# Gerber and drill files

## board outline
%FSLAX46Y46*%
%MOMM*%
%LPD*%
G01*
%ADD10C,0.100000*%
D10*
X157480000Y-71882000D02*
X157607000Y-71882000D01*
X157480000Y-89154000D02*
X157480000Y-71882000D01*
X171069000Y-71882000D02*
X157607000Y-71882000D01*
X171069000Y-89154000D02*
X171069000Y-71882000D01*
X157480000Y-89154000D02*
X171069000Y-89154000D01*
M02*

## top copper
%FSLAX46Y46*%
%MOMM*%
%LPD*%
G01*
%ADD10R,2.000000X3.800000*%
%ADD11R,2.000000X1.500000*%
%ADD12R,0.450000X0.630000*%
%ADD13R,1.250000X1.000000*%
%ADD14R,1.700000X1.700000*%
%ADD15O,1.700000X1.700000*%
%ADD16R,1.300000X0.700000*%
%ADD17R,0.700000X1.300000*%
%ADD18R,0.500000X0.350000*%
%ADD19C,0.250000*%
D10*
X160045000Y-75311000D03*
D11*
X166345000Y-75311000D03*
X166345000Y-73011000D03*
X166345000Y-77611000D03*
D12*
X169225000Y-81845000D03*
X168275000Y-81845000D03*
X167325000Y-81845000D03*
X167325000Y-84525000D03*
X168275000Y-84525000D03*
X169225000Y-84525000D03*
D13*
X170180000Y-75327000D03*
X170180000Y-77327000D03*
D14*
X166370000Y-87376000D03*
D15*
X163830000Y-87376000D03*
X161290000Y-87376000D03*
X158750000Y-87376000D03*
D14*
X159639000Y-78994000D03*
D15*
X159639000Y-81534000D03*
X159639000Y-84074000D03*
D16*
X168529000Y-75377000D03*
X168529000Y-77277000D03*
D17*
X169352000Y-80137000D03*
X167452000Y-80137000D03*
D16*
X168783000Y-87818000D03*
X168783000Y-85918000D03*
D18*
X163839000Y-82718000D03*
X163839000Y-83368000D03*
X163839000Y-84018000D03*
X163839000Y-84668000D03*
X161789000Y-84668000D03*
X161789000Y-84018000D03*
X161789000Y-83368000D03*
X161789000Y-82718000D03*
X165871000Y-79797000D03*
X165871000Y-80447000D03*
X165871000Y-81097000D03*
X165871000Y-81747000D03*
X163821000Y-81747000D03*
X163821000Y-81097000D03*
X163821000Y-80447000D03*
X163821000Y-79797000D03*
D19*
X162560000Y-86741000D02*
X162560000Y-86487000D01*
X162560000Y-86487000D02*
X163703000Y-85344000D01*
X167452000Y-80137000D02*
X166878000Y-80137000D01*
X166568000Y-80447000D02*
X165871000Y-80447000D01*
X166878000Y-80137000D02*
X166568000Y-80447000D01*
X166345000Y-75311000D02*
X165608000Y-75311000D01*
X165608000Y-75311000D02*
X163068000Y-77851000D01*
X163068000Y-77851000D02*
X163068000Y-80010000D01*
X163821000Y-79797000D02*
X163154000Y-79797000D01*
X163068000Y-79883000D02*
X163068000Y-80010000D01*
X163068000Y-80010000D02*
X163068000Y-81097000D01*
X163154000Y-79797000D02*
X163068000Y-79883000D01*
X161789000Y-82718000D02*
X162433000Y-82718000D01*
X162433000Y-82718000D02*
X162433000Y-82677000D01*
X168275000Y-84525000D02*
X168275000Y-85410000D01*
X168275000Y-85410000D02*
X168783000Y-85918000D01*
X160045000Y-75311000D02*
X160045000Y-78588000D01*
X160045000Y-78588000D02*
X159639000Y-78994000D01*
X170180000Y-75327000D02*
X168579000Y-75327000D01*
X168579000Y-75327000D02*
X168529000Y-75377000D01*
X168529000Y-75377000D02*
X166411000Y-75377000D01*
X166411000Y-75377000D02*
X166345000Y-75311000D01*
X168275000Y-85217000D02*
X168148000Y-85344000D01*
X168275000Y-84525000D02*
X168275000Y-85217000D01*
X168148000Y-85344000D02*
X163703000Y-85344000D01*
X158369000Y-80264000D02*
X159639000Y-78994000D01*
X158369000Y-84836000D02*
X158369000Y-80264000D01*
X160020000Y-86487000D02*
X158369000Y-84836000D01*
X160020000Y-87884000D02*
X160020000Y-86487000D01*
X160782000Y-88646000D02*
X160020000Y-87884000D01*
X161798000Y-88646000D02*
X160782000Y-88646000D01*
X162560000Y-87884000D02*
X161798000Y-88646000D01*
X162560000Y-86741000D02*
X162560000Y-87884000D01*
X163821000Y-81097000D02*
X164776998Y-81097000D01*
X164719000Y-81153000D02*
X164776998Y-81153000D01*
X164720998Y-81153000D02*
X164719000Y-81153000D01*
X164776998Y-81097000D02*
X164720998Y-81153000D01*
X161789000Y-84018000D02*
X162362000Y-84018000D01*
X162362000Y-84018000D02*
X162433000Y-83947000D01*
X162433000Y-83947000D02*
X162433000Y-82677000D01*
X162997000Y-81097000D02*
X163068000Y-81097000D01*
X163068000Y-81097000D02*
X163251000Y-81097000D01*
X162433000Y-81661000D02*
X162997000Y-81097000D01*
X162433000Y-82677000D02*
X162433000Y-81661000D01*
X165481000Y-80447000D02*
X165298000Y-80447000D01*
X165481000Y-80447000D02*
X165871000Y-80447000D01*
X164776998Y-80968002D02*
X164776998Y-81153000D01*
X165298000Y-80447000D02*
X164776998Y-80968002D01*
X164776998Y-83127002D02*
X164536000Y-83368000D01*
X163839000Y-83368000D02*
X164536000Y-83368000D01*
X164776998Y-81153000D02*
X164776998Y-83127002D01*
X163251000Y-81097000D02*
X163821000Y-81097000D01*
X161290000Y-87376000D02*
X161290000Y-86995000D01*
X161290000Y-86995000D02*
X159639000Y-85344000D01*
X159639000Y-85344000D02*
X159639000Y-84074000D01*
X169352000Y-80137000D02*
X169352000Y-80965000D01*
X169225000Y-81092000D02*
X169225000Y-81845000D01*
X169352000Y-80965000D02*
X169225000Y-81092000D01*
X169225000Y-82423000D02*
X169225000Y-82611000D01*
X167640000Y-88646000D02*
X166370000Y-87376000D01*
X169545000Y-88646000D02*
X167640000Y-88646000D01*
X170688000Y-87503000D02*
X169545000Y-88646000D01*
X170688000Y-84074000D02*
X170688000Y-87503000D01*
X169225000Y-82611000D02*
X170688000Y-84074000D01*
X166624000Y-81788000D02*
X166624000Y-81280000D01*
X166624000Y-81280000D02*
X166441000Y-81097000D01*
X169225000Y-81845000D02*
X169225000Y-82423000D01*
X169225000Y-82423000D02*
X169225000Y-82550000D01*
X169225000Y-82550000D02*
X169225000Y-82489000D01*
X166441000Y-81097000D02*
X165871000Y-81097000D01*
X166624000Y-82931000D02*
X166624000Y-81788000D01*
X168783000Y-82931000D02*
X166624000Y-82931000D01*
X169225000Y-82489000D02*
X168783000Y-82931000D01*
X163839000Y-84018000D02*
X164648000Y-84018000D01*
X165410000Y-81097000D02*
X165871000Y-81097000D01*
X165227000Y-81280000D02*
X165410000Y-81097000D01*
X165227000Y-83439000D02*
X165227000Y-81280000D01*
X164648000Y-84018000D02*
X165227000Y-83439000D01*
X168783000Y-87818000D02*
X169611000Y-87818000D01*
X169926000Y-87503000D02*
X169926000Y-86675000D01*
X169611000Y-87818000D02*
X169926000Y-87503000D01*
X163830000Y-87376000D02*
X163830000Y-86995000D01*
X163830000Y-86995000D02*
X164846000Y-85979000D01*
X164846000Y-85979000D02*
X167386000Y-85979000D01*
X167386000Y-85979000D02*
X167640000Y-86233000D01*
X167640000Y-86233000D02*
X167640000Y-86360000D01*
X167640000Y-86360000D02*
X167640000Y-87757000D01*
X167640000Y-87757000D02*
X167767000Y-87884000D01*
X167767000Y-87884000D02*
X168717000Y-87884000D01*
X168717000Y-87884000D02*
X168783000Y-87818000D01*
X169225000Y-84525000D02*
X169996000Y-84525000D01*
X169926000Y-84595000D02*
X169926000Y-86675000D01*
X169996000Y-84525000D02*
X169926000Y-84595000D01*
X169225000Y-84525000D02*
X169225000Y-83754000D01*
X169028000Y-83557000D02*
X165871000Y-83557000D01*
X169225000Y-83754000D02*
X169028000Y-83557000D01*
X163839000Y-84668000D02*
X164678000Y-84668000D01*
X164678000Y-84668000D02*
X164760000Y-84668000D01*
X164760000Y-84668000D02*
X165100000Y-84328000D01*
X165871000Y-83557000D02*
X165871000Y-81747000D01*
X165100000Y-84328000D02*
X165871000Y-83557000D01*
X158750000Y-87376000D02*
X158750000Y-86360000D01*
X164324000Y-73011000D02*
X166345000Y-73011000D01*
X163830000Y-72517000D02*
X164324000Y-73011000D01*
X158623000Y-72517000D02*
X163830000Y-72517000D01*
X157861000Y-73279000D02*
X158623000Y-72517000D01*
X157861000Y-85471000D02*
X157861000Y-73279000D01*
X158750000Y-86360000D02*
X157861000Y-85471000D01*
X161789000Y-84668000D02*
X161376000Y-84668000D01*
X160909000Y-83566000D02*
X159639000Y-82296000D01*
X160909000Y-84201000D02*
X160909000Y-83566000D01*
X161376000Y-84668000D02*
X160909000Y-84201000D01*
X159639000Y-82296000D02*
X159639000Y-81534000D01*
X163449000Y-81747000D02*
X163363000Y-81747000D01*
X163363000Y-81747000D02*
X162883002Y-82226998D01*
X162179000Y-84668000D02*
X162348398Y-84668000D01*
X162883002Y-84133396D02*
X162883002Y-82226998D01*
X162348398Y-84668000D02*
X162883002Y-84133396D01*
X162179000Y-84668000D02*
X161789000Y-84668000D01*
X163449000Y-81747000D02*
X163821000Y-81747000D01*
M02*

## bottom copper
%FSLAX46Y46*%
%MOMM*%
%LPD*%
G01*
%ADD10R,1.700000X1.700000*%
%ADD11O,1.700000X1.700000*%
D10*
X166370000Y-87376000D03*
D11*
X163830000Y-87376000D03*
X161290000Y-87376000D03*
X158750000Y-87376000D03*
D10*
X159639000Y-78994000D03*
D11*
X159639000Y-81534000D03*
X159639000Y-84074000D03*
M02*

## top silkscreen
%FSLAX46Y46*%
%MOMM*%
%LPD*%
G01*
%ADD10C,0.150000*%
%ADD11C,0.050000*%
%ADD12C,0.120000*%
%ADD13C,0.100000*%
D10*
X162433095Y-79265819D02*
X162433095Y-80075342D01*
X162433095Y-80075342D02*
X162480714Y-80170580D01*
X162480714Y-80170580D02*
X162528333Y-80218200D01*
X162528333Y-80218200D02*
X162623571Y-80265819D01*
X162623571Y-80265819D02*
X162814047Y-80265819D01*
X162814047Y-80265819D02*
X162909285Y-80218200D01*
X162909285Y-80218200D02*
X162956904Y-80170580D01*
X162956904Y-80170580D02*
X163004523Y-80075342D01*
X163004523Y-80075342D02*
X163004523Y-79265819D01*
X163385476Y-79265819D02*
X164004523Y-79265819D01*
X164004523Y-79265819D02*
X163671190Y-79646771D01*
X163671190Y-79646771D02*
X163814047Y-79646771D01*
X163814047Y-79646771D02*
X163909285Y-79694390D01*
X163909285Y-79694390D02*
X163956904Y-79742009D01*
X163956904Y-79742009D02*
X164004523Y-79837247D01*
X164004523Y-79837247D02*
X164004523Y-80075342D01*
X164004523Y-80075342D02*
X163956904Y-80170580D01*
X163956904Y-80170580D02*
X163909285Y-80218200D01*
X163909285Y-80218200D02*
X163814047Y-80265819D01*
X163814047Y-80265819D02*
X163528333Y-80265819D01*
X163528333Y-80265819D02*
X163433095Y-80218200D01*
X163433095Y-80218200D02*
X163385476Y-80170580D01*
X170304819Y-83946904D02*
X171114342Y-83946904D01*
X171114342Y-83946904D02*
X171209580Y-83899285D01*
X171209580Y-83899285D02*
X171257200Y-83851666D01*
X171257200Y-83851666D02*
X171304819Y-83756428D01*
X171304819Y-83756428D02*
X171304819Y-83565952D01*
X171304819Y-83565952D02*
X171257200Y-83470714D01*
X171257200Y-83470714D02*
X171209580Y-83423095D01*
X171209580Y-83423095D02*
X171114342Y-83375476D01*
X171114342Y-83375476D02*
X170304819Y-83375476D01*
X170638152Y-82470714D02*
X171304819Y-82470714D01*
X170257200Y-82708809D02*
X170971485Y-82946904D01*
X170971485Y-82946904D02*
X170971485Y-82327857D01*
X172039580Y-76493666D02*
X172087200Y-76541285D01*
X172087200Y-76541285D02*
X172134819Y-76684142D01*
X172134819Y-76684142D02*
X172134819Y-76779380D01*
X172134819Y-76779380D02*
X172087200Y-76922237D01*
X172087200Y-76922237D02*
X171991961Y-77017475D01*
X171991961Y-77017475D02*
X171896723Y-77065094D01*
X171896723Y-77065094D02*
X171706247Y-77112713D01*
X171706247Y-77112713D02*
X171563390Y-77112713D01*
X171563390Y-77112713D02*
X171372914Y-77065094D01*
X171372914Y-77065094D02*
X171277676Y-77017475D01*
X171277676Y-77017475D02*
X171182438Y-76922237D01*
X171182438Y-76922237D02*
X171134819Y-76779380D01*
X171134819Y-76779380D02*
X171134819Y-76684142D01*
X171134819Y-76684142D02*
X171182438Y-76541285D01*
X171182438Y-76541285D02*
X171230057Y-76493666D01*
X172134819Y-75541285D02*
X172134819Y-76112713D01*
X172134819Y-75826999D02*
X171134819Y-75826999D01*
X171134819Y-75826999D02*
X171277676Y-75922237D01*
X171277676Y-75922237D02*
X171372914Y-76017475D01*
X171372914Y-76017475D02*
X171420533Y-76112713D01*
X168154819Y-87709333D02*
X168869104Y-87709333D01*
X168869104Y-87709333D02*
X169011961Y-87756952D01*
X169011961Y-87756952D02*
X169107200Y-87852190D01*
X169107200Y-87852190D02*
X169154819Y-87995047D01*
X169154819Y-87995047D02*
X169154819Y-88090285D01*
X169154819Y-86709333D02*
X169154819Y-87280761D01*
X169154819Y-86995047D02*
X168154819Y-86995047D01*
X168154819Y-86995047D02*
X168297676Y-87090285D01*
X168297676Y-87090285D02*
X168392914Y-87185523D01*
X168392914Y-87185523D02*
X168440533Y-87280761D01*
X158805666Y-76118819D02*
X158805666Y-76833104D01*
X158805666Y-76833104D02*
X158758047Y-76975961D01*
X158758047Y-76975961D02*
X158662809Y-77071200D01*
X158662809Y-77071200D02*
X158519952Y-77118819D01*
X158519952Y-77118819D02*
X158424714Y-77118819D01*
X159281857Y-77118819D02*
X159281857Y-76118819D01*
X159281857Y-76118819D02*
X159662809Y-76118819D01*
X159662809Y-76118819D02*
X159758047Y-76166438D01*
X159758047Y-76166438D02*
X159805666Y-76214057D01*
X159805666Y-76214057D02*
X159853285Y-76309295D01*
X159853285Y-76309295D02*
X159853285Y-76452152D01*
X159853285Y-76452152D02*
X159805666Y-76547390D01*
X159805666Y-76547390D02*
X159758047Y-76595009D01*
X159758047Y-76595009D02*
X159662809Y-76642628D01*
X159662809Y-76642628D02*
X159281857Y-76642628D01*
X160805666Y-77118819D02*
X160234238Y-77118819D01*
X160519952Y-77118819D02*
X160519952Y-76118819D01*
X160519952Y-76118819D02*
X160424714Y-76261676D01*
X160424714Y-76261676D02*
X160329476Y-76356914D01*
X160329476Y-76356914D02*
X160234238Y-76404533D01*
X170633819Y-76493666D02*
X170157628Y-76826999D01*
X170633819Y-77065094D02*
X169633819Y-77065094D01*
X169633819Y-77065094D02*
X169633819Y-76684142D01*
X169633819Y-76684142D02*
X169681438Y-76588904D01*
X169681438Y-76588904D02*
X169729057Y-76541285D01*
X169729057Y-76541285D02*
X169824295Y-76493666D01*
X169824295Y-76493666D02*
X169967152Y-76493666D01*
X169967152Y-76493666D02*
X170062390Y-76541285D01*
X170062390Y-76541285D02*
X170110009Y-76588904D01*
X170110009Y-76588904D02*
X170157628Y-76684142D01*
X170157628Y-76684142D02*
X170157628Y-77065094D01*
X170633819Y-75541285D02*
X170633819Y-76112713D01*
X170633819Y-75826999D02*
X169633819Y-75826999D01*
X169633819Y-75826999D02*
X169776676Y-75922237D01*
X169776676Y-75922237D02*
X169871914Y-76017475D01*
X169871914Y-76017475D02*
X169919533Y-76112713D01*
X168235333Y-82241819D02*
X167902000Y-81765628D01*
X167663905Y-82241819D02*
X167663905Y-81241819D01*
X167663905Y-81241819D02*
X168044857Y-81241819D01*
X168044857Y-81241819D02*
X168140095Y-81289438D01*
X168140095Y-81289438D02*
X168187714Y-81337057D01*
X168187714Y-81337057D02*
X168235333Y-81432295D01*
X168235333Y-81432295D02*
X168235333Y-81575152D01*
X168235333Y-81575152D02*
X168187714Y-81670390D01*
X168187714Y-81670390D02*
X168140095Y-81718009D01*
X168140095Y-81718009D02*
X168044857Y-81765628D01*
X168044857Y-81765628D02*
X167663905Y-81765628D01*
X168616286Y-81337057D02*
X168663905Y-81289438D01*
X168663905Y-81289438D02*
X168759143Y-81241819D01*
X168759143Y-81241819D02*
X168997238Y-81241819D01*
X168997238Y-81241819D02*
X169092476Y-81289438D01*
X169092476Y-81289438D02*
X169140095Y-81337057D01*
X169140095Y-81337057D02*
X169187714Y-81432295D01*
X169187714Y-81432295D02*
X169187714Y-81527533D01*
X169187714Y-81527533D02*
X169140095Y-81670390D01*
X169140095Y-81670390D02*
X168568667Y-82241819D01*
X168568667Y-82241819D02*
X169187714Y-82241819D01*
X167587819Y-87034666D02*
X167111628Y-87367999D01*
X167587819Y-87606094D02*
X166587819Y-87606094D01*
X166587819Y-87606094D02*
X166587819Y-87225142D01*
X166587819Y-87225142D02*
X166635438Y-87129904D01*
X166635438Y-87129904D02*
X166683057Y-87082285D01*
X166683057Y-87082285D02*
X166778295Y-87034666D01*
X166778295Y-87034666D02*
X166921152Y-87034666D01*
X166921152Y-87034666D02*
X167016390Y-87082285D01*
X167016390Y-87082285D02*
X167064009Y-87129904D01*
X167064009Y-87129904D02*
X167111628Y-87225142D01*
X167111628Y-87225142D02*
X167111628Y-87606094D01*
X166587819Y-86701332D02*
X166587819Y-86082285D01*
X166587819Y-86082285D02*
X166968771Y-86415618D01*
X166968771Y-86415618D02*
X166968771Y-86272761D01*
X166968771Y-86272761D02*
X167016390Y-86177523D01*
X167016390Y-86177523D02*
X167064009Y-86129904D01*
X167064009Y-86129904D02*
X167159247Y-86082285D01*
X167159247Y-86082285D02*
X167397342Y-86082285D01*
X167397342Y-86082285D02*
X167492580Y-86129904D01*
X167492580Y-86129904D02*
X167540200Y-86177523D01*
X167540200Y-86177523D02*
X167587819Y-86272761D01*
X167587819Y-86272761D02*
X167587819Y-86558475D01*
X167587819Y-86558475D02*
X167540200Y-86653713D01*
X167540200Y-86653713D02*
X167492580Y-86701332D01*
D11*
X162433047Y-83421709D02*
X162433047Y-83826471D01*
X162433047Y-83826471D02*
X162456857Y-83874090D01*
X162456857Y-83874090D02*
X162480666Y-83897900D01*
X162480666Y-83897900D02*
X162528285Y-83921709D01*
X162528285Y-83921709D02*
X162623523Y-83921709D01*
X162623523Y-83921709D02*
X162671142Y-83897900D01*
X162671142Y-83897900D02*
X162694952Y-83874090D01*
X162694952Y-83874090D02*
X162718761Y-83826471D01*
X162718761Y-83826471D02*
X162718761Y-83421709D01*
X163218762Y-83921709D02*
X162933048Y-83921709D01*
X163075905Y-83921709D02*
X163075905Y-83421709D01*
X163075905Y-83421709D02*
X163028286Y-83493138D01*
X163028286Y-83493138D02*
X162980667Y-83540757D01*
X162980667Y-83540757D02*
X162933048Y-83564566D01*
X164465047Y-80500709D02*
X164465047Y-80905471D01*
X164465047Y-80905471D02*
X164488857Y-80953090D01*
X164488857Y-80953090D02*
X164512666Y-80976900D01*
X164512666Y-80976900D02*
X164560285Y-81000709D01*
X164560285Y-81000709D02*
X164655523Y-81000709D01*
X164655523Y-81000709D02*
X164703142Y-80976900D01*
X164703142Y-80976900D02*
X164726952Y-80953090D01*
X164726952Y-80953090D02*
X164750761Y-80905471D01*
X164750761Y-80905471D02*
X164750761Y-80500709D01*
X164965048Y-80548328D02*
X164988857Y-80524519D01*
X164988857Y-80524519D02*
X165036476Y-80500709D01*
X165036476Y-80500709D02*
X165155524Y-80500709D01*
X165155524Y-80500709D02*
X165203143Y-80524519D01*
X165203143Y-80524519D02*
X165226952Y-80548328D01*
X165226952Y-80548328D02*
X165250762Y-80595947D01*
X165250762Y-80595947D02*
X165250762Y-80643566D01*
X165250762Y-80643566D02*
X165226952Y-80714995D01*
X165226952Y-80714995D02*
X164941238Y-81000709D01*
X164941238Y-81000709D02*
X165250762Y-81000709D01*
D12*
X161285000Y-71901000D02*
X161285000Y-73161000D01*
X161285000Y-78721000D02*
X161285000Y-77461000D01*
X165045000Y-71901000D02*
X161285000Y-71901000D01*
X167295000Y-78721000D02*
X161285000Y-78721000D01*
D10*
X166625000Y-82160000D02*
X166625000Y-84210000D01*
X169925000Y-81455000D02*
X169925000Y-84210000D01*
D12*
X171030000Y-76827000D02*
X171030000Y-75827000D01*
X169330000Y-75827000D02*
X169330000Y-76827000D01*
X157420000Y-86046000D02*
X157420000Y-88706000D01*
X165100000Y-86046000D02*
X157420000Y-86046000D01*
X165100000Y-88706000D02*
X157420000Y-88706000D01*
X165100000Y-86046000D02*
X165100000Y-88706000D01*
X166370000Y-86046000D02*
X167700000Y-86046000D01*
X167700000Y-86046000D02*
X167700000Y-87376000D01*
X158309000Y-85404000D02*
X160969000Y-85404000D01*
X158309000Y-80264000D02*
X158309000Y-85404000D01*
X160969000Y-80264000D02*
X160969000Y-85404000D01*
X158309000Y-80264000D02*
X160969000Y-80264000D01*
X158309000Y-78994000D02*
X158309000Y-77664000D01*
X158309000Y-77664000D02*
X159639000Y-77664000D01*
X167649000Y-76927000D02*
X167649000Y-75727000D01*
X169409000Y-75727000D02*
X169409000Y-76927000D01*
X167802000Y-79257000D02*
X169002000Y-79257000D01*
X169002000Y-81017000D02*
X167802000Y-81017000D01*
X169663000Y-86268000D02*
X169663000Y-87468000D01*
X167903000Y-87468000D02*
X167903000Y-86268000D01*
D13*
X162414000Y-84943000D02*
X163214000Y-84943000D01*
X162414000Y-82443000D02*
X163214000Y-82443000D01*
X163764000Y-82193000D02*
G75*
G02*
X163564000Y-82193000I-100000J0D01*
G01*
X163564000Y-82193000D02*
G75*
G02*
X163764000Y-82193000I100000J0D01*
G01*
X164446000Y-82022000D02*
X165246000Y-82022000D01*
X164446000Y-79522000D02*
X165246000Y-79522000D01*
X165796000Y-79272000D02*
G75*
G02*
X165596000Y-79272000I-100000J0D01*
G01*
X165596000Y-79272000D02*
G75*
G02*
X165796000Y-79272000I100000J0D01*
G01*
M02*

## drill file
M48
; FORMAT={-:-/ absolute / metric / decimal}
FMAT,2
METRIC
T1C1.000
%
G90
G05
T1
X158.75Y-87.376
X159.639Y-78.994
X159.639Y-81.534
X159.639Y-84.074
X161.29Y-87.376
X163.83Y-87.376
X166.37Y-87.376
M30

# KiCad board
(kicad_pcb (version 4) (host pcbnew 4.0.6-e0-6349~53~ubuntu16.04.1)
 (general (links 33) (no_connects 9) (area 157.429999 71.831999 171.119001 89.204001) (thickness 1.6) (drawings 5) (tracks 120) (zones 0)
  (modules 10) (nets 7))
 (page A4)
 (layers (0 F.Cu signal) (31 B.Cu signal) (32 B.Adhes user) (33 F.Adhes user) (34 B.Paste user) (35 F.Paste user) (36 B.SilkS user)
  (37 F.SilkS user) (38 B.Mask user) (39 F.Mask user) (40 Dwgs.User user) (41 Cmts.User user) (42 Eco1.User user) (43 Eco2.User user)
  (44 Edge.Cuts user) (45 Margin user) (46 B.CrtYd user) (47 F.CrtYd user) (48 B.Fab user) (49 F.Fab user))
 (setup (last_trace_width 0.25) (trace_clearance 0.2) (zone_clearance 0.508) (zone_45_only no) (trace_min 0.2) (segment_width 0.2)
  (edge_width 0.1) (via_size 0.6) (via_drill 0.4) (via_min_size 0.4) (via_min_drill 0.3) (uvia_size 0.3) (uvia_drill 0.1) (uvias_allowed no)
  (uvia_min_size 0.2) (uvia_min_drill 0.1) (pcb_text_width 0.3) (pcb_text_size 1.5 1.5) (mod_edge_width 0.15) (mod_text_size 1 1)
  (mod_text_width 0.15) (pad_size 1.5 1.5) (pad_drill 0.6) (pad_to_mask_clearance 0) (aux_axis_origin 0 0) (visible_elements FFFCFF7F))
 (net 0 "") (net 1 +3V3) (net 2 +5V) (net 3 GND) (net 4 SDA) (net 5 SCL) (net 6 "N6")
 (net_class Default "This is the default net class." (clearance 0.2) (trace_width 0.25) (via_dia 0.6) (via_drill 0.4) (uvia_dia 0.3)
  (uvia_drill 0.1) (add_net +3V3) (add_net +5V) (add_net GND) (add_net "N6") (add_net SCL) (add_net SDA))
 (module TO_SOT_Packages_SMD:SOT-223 (layer F.Cu) (at 163.195 75.311 180)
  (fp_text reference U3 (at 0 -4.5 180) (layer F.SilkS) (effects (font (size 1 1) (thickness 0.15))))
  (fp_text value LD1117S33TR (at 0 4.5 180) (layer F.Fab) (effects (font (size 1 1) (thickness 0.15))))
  (fp_line (start 1.91 3.41) (end 1.91 2.15) (layer F.SilkS) (width 0.12))
  (fp_line (start 1.91 -3.41) (end 1.91 -2.15) (layer F.SilkS) (width 0.12))
  (fp_line (start -1.85 3.41) (end 1.91 3.41) (layer F.SilkS) (width 0.12))
  (fp_line (start -4.1 -3.41) (end 1.91 -3.41) (layer F.SilkS) (width 0.12))
  (pad 2 smd rect (at 3.15 0 180) (size 2 3.8) (layers F.Cu F.Paste F.Mask) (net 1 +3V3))
  (pad 2 smd rect (at -3.15 0 180) (size 2 1.5) (layers F.Cu F.Paste F.Mask) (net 1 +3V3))
  (pad 3 smd rect (at -3.15 2.3 180) (size 2 1.5) (layers F.Cu F.Paste F.Mask) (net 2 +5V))
  (pad 1 smd rect (at -3.15 -2.3 180) (size 2 1.5) (layers F.Cu F.Paste F.Mask) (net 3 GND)))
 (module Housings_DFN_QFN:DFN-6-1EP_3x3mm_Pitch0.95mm (layer F.Cu) (at 168.275 83.185 270)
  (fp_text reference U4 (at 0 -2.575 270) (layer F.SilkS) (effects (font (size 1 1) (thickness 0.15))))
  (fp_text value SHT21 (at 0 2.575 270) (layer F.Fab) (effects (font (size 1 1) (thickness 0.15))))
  (fp_line (start -1.025 1.65) (end 1.025 1.65) (layer F.SilkS) (width 0.15))
  (fp_line (start -1.73 -1.65) (end 1.025 -1.65) (layer F.SilkS) (width 0.15))
  (pad 1 smd rect (at -1.34 -0.95 270) (size 0.63 0.45) (layers F.Cu F.Paste F.Mask) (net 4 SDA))
  (pad 2 smd rect (at -1.34 0 270) (size 0.63 0.45) (layers F.Cu F.Paste F.Mask) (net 3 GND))
  (pad 3 smd rect (at -1.34 0.95 270) (size 0.63 0.45) (layers F.Cu F.Paste F.Mask))
  (pad 4 smd rect (at 1.34 0.95 270) (size 0.63 0.45) (layers F.Cu F.Paste F.Mask))
  (pad 5 smd rect (at 1.34 0 270) (size 0.63 0.45) (layers F.Cu F.Paste F.Mask) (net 1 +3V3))
  (pad 6 smd rect (at 1.34 -0.95 270) (size 0.63 0.45) (layers F.Cu F.Paste F.Mask) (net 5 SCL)))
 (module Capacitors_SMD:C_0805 (layer F.Cu) (at 170.18 76.327 270)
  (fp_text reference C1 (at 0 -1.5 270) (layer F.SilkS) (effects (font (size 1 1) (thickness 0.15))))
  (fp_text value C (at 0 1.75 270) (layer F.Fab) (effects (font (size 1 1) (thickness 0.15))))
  (fp_line (start 0.5 -0.85) (end -0.5 -0.85) (layer F.SilkS) (width 0.12))
  (fp_line (start -0.5 0.85) (end 0.5 0.85) (layer F.SilkS) (width 0.12))
  (pad 1 smd rect (at -1 0 270) (size 1 1.25) (layers F.Cu F.Paste F.Mask) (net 1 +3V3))
  (pad 2 smd rect (at 1 0 270) (size 1 1.25) (layers F.Cu F.Paste F.Mask) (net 3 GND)))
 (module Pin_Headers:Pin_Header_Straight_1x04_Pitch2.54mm (layer F.Cu) (at 166.37 87.376 270)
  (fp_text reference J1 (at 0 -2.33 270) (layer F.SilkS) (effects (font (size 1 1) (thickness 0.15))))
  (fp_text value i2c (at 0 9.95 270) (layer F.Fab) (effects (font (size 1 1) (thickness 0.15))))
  (fp_line (start -1.33 8.95) (end 1.33 8.95) (layer F.SilkS) (width 0.12))
  (fp_line (start -1.33 1.27) (end -1.33 8.95) (layer F.SilkS) (width 0.12))
  (fp_line (start 1.33 1.27) (end 1.33 8.95) (layer F.SilkS) (width 0.12))
  (fp_line (start -1.33 1.27) (end 1.33 1.27) (layer F.SilkS) (width 0.12))
  (fp_line (start -1.33 0) (end -1.33 -1.33) (layer F.SilkS) (width 0.12))
  (fp_line (start -1.33 -1.33) (end 0 -1.33) (layer F.SilkS) (width 0.12))
  (pad 1 thru_hole rect (at 0 0 270) (size 1.7 1.7) (drill 1) (layers *.Cu *.Mask) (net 4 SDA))
  (pad 2 thru_hole oval (at 0 2.54 270) (size 1.7 1.7) (drill 1) (layers *.Cu *.Mask) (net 5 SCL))
  (pad 3 thru_hole oval (at 0 5.08 270) (size 1.7 1.7) (drill 1) (layers *.Cu *.Mask) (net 3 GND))
  (pad 4 thru_hole oval (at 0 7.62 270) (size 1.7 1.7) (drill 1) (layers *.Cu *.Mask) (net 2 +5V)))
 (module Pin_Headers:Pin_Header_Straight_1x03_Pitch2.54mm (layer F.Cu) (at 159.639 78.994)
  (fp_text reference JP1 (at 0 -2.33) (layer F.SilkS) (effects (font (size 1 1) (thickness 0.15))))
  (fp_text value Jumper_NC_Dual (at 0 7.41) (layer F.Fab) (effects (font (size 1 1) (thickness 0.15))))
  (fp_line (start -1.33 6.41) (end 1.33 6.41) (layer F.SilkS) (width 0.12))
  (fp_line (start -1.33 1.27) (end -1.33 6.41) (layer F.SilkS) (width 0.12))
  (fp_line (start 1.33 1.27) (end 1.33 6.41) (layer F.SilkS) (width 0.12))
  (fp_line (start -1.33 1.27) (end 1.33 1.27) (layer F.SilkS) (width 0.12))
  (fp_line (start -1.33 0) (end -1.33 -1.33) (layer F.SilkS) (width 0.12))
  (fp_line (start -1.33 -1.33) (end 0 -1.33) (layer F.SilkS) (width 0.12))
  (pad 1 thru_hole rect (at 0 0) (size 1.7 1.7) (drill 1) (layers *.Cu *.Mask) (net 1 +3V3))
  (pad 2 thru_hole oval (at 0 2.54) (size 1.7 1.7) (drill 1) (layers *.Cu *.Mask) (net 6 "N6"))
  (pad 3 thru_hole oval (at 0 5.08) (size 1.7 1.7) (drill 1) (layers *.Cu *.Mask) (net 3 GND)))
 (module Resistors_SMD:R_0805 (layer F.Cu) (at 168.529 76.327 270)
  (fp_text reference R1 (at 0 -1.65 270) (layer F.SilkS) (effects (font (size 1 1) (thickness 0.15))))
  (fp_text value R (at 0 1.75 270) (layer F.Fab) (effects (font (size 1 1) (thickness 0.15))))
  (fp_line (start 0.6 0.88) (end -0.6 0.88) (layer F.SilkS) (width 0.12))
  (fp_line (start -0.6 -0.88) (end 0.6 -0.88) (layer F.SilkS) (width 0.12))
  (pad 1 smd rect (at -0.95 0 270) (size 0.7 1.3) (layers F.Cu F.Paste F.Mask) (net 1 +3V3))
  (pad 2 smd rect (at 0.95 0 270) (size 0.7 1.3) (layers F.Cu F.Paste F.Mask) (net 3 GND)))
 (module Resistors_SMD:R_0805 (layer F.Cu) (at 168.402 80.137 180)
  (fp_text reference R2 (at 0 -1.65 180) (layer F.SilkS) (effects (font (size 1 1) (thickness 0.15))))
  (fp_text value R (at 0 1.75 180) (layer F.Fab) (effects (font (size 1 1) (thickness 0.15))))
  (fp_line (start 0.6 0.88) (end -0.6 0.88) (layer F.SilkS) (width 0.12))
  (fp_line (start -0.6 -0.88) (end 0.6 -0.88) (layer F.SilkS) (width 0.12))
  (pad 1 smd rect (at -0.95 0 180) (size 0.7 1.3) (layers F.Cu F.Paste F.Mask) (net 4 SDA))
  (pad 2 smd rect (at 0.95 0 180) (size 0.7 1.3) (layers F.Cu F.Paste F.Mask) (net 1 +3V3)))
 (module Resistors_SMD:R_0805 (layer F.Cu) (at 168.783 86.868 90)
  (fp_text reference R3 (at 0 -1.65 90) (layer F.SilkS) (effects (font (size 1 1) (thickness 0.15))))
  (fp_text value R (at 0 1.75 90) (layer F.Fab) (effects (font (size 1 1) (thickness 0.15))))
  (fp_line (start 0.6 0.88) (end -0.6 0.88) (layer F.SilkS) (width 0.12))
  (fp_line (start -0.6 -0.88) (end 0.6 -0.88) (layer F.SilkS) (width 0.12))
  (pad 1 smd rect (at -0.95 0 90) (size 0.7 1.3) (layers F.Cu F.Paste F.Mask) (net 5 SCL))
  (pad 2 smd rect (at 0.95 0 90) (size 0.7 1.3) (layers F.Cu F.Paste F.Mask) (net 1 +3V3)))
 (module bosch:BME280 (layer F.Cu) (at 162.814 83.693)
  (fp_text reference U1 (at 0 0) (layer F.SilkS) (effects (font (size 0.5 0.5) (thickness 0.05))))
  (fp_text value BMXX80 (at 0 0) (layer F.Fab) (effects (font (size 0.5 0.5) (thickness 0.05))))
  (fp_line (start -0.4 1.25) (end 0.4 1.25) (layer F.SilkS) (width 0.1))
  (fp_line (start -0.4 -1.25) (end 0.4 -1.25) (layer F.SilkS) (width 0.1))
  (fp_circle (center 0.85 -1.5) (end 0.85 -1.6) (layer F.SilkS) (width 0.1))
  (pad 1 smd rect (at 1.025 -0.975) (size 0.5 0.35) (layers F.Cu F.Paste F.Mask) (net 3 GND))
  (pad 2 smd rect (at 1.025 -0.325) (size 0.5 0.35) (layers F.Cu F.Paste F.Mask) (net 1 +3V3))
  (pad 3 smd rect (at 1.025 0.325) (size 0.5 0.35) (layers F.Cu F.Paste F.Mask) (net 4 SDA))
  (pad 4 smd rect (at 1.025 0.975) (size 0.5 0.35) (layers F.Cu F.Paste F.Mask) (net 5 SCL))
  (pad 5 smd rect (at -1.025 0.975) (size 0.5 0.35) (layers F.Cu F.Paste F.Mask) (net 6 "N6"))
  (pad 6 smd rect (at -1.025 0.325) (size 0.5 0.35) (layers F.Cu F.Paste F.Mask) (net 1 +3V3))
  (pad 7 smd rect (at -1.025 -0.325) (size 0.5 0.35) (layers F.Cu F.Paste F.Mask) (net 3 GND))
  (pad 8 smd rect (at -1.025 -0.975) (size 0.5 0.35) (layers F.Cu F.Paste F.Mask) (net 1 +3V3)))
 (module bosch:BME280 (layer F.Cu) (at 164.846 80.772)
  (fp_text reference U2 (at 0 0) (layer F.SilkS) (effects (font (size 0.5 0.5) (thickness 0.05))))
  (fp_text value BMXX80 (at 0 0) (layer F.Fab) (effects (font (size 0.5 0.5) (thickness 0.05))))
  (fp_line (start -0.4 1.25) (end 0.4 1.25) (layer F.SilkS) (width 0.1))
  (fp_line (start -0.4 -1.25) (end 0.4 -1.25) (layer F.SilkS) (width 0.1))
  (fp_circle (center 0.85 -1.5) (end 0.85 -1.6) (layer F.SilkS) (width 0.1))
  (pad 1 smd rect (at 1.025 -0.975) (size 0.5 0.35) (layers F.Cu F.Paste F.Mask) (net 3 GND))
  (pad 2 smd rect (at 1.025 -0.325) (size 0.5 0.35) (layers F.Cu F.Paste F.Mask) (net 1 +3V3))
  (pad 3 smd rect (at 1.025 0.325) (size 0.5 0.35) (layers F.Cu F.Paste F.Mask) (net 4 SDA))
  (pad 4 smd rect (at 1.025 0.975) (size 0.5 0.35) (layers F.Cu F.Paste F.Mask) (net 5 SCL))
  (pad 5 smd rect (at -1.025 0.975) (size 0.5 0.35) (layers F.Cu F.Paste F.Mask) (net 6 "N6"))
  (pad 6 smd rect (at -1.025 0.325) (size 0.5 0.35) (layers F.Cu F.Paste F.Mask) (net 1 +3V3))
  (pad 7 smd rect (at -1.025 -0.325) (size 0.5 0.35) (layers F.Cu F.Paste F.Mask) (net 3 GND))
  (pad 8 smd rect (at -1.025 -0.975) (size 0.5 0.35) (layers F.Cu F.Paste F.Mask) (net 1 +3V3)))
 (gr_line (start 157.48 71.882) (end 157.607 71.882) (angle 90) (layer Edge.Cuts) (width 0.1))
 (gr_line (start 157.48 89.154) (end 157.48 71.882) (angle 90) (layer Edge.Cuts) (width 0.1))
 (gr_line (start 171.069 71.882) (end 157.607 71.882) (angle 90) (layer Edge.Cuts) (width 0.1))
 (gr_line (start 171.069 89.154) (end 171.069 71.882) (angle 90) (layer Edge.Cuts) (width 0.1))
 (gr_line (start 157.48 89.154) (end 171.069 89.154) (angle 90) (layer Edge.Cuts) (width 0.1))
 (segment (start 162.56 86.741) (end 162.56 86.487) (width 0.25) (layer F.Cu) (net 1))
 (segment (start 162.56 86.487) (end 163.703 85.344) (width 0.25) (layer F.Cu) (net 1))
 (segment (start 167.452 80.137) (end 166.878 80.137) (width 0.25) (layer F.Cu) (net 1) (status 400000))
 (segment (start 166.568 80.447) (end 165.871 80.447) (width 0.25) (layer F.Cu) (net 1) (status 800000))
 (segment (start 166.878 80.137) (end 166.568 80.447) (width 0.25) (layer F.Cu) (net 1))
 (segment (start 166.345 75.311) (end 165.608 75.311) (width 0.25) (layer F.Cu) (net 1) (status C00000))
 (segment (start 165.608 75.311) (end 163.068 77.851) (width 0.25) (layer F.Cu) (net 1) (status 400000))
 (segment (start 163.068 77.851) (end 163.068 80.01) (width 0.25) (layer F.Cu) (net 1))
 (segment (start 163.821 79.797) (end 163.154 79.797) (width 0.25) (layer F.Cu) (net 1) (status 400000))
 (segment (start 163.068 79.883) (end 163.068 80.01) (width 0.25) (layer F.Cu) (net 1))
 (segment (start 163.068 80.01) (end 163.068 81.097) (width 0.25) (layer F.Cu) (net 1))
 (segment (start 163.154 79.797) (end 163.068 79.883) (width 0.25) (layer F.Cu) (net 1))
 (segment (start 161.789 82.718) (end 162.433 82.718) (width 0.25) (layer F.Cu) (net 1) (status 400000))
 (segment (start 162.433 82.718) (end 162.433 82.677) (width 0.25) (layer F.Cu) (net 1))
 (segment (start 168.275 84.525) (end 168.275 85.41) (width 0.25) (layer F.Cu) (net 1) (status 400000))
 (segment (start 168.275 85.41) (end 168.783 85.918) (width 0.25) (layer F.Cu) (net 1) (status 800000))
 (segment (start 160.045 75.311) (end 160.045 78.588) (width 0.25) (layer F.Cu) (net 1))
 (segment (start 160.045 78.588) (end 159.639 78.994) (width 0.25) (layer F.Cu) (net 1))
 (segment (start 170.18 75.327) (end 168.579 75.327) (width 0.25) (layer F.Cu) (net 1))
 (segment (start 168.579 75.327) (end 168.529 75.377) (width 0.25) (layer F.Cu) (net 1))
 (segment (start 168.529 75.377) (end 166.411 75.377) (width 0.25) (layer F.Cu) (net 1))
 (segment (start 166.411 75.377) (end 166.345 75.311) (width 0.25) (layer F.Cu) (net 1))
 (segment (start 168.275 85.217) (end 168.148 85.344) (width 0.25) (layer F.Cu) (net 1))
 (segment (start 168.275 84.525) (end 168.275 85.217) (width 0.25) (layer F.Cu) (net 1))
 (segment (start 168.148 85.344) (end 163.703 85.344) (width 0.25) (layer F.Cu) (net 1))
 (segment (start 158.369 80.264) (end 159.639 78.994) (width 0.25) (layer F.Cu) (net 1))
 (segment (start 158.369 84.836) (end 158.369 80.264) (width 0.25) (layer F.Cu) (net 1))
 (segment (start 160.02 86.487) (end 158.369 84.836) (width 0.25) (layer F.Cu) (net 1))
 (segment (start 160.02 87.884) (end 160.02 86.487) (width 0.25) (layer F.Cu) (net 1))
 (segment (start 160.782 88.646) (end 160.02 87.884) (width 0.25) (layer F.Cu) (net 1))
 (segment (start 161.798 88.646) (end 160.782 88.646) (width 0.25) (layer F.Cu) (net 1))
 (segment (start 162.56 87.884) (end 161.798 88.646) (width 0.25) (layer F.Cu) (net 1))
 (segment (start 162.56 86.741) (end 162.56 87.884) (width 0.25) (layer F.Cu) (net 1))
 (segment (start 163.821 81.097) (end 164.776998 81.097) (width 0.25) (layer F.Cu) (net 1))
 (segment (start 164.719 81.153) (end 164.776998 81.153) (width 0.25) (layer F.Cu) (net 1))
 (segment (start 164.720998 81.153) (end 164.719 81.153) (width 0.25) (layer F.Cu) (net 1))
 (segment (start 164.776998 81.097) (end 164.720998 81.153) (width 0.25) (layer F.Cu) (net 1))
 (segment (start 161.789 84.018) (end 162.362 84.018) (width 0.25) (layer F.Cu) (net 1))
 (segment (start 162.362 84.018) (end 162.433 83.947) (width 0.25) (layer F.Cu) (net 1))
 (segment (start 162.433 83.947) (end 162.433 82.677) (width 0.25) (layer F.Cu) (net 1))
 (segment (start 162.997 81.097) (end 163.068 81.097) (width 0.25) (layer F.Cu) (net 1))
 (segment (start 163.068 81.097) (end 163.251 81.097) (width 0.25) (layer F.Cu) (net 1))
 (segment (start 162.433 81.661) (end 162.997 81.097) (width 0.25) (layer F.Cu) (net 1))
 (segment (start 162.433 82.677) (end 162.433 81.661) (width 0.25) (layer F.Cu) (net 1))
 (segment (start 165.481 80.447) (end 165.298 80.447) (width 0.25) (layer F.Cu) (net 1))
 (segment (start 165.481 80.447) (end 165.871 80.447) (width 0.25) (layer F.Cu) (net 1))
 (segment (start 164.776998 80.968002) (end 164.776998 81.153) (width 0.25) (layer F.Cu) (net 1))
 (segment (start 165.298 80.447) (end 164.776998 80.968002) (width 0.25) (layer F.Cu) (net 1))
 (segment (start 164.776998 83.127002) (end 164.536 83.368) (width 0.25) (layer F.Cu) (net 1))
 (segment (start 163.839 83.368) (end 164.536 83.368) (width 0.25) (layer F.Cu) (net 1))
 (segment (start 164.776998 81.153) (end 164.776998 83.127002) (width 0.25) (layer F.Cu) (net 1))
 (segment (start 163.251 81.097) (end 163.821 81.097) (width 0.25) (layer F.Cu) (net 1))
 (segment (start 161.29 87.376) (end 161.29 86.995) (width 0.25) (layer F.Cu) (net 3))
 (segment (start 161.29 86.995) (end 159.639 85.344) (width 0.25) (layer F.Cu) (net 3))
 (segment (start 159.639 85.344) (end 159.639 84.074) (width 0.25) (layer F.Cu) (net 3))
 (segment (start 169.352 80.137) (end 169.352 80.965) (width 0.25) (layer F.Cu) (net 4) (status 400000))
 (segment (start 169.225 81.092) (end 169.225 81.845) (width 0.25) (layer F.Cu) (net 4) (status 800000))
 (segment (start 169.352 80.965) (end 169.225 81.092) (width 0.25) (layer F.Cu) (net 4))
 (segment (start 169.225 82.423) (end 169.225 82.611) (width 0.25) (layer F.Cu) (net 4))
 (segment (start 167.64 88.646) (end 166.37 87.376) (width 0.25) (layer F.Cu) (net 4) (status 800000))
 (segment (start 169.545 88.646) (end 167.64 88.646) (width 0.25) (layer F.Cu) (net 4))
 (segment (start 170.688 87.503) (end 169.545 88.646) (width 0.25) (layer F.Cu) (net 4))
 (segment (start 170.688 84.074) (end 170.688 87.503) (width 0.25) (layer F.Cu) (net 4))
 (segment (start 169.225 82.611) (end 170.688 84.074) (width 0.25) (layer F.Cu) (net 4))
 (segment (start 166.624 81.788) (end 166.624 81.28) (width 0.25) (layer F.Cu) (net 4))
 (segment (start 166.624 81.28) (end 166.441 81.097) (width 0.25) (layer F.Cu) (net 4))
 (segment (start 169.225 81.845) (end 169.225 82.423) (width 0.25) (layer F.Cu) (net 4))
 (segment (start 169.225 82.423) (end 169.225 82.55) (width 0.25) (layer F.Cu) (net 4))
 (segment (start 169.225 82.55) (end 169.225 82.489) (width 0.25) (layer F.Cu) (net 4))
 (segment (start 166.441 81.097) (end 165.871 81.097) (width 0.25) (layer F.Cu) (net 4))
 (segment (start 166.624 82.931) (end 166.624 81.788) (width 0.25) (layer F.Cu) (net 4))
 (segment (start 168.783 82.931) (end 166.624 82.931) (width 0.25) (layer F.Cu) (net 4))
 (segment (start 169.225 82.489) (end 168.783 82.931) (width 0.25) (layer F.Cu) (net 4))
 (segment (start 163.839 84.018) (end 164.648 84.018) (width 0.25) (layer F.Cu) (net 4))
 (segment (start 165.41 81.097) (end 165.871 81.097) (width 0.25) (layer F.Cu) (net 4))
 (segment (start 165.227 81.28) (end 165.41 81.097) (width 0.25) (layer F.Cu) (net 4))
 (segment (start 165.227 83.439) (end 165.227 81.28) (width 0.25) (layer F.Cu) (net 4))
 (segment (start 164.648 84.018) (end 165.227 83.439) (width 0.25) (layer F.Cu) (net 4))
 (segment (start 168.783 87.818) (end 169.611 87.818) (width 0.25) (layer F.Cu) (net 5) (status 400000))
 (segment (start 169.926 87.503) (end 169.926 86.675) (width 0.25) (layer F.Cu) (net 5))
 (segment (start 169.611 87.818) (end 169.926 87.503) (width 0.25) (layer F.Cu) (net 5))
 (segment (start 163.83 87.376) (end 163.83 86.995) (width 0.25) (layer F.Cu) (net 5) (status C00000))
 (segment (start 163.83 86.995) (end 164.846 85.979) (width 0.25) (layer F.Cu) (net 5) (status 400000))
 (segment (start 164.846 85.979) (end 167.386 85.979) (width 0.25) (layer F.Cu) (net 5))
 (segment (start 167.386 85.979) (end 167.64 86.233) (width 0.25) (layer F.Cu) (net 5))
 (segment (start 167.64 86.233) (end 167.64 86.36) (width 0.25) (layer F.Cu) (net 5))
 (segment (start 167.64 86.36) (end 167.64 87.757) (width 0.25) (layer F.Cu) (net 5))
 (segment (start 167.64 87.757) (end 167.767 87.884) (width 0.25) (layer F.Cu) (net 5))
 (segment (start 167.767 87.884) (end 168.717 87.884) (width 0.25) (layer F.Cu) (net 5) (status 800000))
 (segment (start 168.717 87.884) (end 168.783 87.818) (width 0.25) (layer F.Cu) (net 5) (status C00000))
 (segment (start 169.225 84.525) (end 169.996 84.525) (width 0.25) (layer F.Cu) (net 5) (status 400000))
 (segment (start 169.926 84.595) (end 169.926 86.675) (width 0.25) (layer F.Cu) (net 5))
 (segment (start 169.996 84.525) (end 169.926 84.595) (width 0.25) (layer F.Cu) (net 5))
 (segment (start 169.225 84.525) (end 169.225 83.754) (width 0.25) (layer F.Cu) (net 5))
 (segment (start 169.028 83.557) (end 165.871 83.557) (width 0.25) (layer F.Cu) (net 5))
 (segment (start 169.225 83.754) (end 169.028 83.557) (width 0.25) (layer F.Cu) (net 5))
 (segment (start 163.839 84.668) (end 164.678 84.668) (width 0.25) (layer F.Cu) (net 5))
 (segment (start 164.678 84.668) (end 164.76 84.668) (width 0.25) (layer F.Cu) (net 5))
 (segment (start 164.76 84.668) (end 165.1 84.328) (width 0.25) (layer F.Cu) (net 5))
 (segment (start 165.871 83.557) (end 165.871 81.747) (width 0.25) (layer F.Cu) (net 5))
 (segment (start 165.1 84.328) (end 165.871 83.557) (width 0.25) (layer F.Cu) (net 5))
 (segment (start 158.75 87.376) (end 158.75 86.36) (width 0.25) (layer F.Cu) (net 2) (status 400000))
 (segment (start 164.324 73.011) (end 166.345 73.011) (width 0.25) (layer F.Cu) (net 2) (status 800000))
 (segment (start 163.83 72.517) (end 164.324 73.011) (width 0.25) (layer F.Cu) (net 2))
 (segment (start 158.623 72.517) (end 163.83 72.517) (width 0.25) (layer F.Cu) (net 2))
 (segment (start 157.861 73.279) (end 158.623 72.517) (width 0.25) (layer F.Cu) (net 2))
 (segment (start 157.861 85.471) (end 157.861 73.279) (width 0.25) (layer F.Cu) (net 2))
 (segment (start 158.75 86.36) (end 157.861 85.471) (width 0.25) (layer F.Cu) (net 2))
 (segment (start 161.789 84.668) (end 161.376 84.668) (width 0.25) (layer F.Cu) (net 6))
 (segment (start 160.909 83.566) (end 159.639 82.296) (width 0.25) (layer F.Cu) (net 6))
 (segment (start 160.909 84.201) (end 160.909 83.566) (width 0.25) (layer F.Cu) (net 6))
 (segment (start 161.376 84.668) (end 160.909 84.201) (width 0.25) (layer F.Cu) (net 6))
 (segment (start 159.639 82.296) (end 159.639 81.534) (width 0.25) (layer F.Cu) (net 6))
 (segment (start 163.449 81.747) (end 163.363 81.747) (width 0.25) (layer F.Cu) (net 6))
 (segment (start 163.363 81.747) (end 162.883002 82.226998) (width 0.25) (layer F.Cu) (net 6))
 (segment (start 162.179 84.668) (end 162.348398 84.668) (width 0.25) (layer F.Cu) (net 6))
 (segment (start 162.883002 84.133396) (end 162.883002 82.226998) (width 0.25) (layer F.Cu) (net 6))
 (segment (start 162.348398 84.668) (end 162.883002 84.133396) (width 0.25) (layer F.Cu) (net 6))
 (segment (start 162.179 84.668) (end 161.789 84.668) (width 0.25) (layer F.Cu) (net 6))
 (segment (start 163.449 81.747) (end 163.821 81.747) (width 0.25) (layer F.Cu) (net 6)))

